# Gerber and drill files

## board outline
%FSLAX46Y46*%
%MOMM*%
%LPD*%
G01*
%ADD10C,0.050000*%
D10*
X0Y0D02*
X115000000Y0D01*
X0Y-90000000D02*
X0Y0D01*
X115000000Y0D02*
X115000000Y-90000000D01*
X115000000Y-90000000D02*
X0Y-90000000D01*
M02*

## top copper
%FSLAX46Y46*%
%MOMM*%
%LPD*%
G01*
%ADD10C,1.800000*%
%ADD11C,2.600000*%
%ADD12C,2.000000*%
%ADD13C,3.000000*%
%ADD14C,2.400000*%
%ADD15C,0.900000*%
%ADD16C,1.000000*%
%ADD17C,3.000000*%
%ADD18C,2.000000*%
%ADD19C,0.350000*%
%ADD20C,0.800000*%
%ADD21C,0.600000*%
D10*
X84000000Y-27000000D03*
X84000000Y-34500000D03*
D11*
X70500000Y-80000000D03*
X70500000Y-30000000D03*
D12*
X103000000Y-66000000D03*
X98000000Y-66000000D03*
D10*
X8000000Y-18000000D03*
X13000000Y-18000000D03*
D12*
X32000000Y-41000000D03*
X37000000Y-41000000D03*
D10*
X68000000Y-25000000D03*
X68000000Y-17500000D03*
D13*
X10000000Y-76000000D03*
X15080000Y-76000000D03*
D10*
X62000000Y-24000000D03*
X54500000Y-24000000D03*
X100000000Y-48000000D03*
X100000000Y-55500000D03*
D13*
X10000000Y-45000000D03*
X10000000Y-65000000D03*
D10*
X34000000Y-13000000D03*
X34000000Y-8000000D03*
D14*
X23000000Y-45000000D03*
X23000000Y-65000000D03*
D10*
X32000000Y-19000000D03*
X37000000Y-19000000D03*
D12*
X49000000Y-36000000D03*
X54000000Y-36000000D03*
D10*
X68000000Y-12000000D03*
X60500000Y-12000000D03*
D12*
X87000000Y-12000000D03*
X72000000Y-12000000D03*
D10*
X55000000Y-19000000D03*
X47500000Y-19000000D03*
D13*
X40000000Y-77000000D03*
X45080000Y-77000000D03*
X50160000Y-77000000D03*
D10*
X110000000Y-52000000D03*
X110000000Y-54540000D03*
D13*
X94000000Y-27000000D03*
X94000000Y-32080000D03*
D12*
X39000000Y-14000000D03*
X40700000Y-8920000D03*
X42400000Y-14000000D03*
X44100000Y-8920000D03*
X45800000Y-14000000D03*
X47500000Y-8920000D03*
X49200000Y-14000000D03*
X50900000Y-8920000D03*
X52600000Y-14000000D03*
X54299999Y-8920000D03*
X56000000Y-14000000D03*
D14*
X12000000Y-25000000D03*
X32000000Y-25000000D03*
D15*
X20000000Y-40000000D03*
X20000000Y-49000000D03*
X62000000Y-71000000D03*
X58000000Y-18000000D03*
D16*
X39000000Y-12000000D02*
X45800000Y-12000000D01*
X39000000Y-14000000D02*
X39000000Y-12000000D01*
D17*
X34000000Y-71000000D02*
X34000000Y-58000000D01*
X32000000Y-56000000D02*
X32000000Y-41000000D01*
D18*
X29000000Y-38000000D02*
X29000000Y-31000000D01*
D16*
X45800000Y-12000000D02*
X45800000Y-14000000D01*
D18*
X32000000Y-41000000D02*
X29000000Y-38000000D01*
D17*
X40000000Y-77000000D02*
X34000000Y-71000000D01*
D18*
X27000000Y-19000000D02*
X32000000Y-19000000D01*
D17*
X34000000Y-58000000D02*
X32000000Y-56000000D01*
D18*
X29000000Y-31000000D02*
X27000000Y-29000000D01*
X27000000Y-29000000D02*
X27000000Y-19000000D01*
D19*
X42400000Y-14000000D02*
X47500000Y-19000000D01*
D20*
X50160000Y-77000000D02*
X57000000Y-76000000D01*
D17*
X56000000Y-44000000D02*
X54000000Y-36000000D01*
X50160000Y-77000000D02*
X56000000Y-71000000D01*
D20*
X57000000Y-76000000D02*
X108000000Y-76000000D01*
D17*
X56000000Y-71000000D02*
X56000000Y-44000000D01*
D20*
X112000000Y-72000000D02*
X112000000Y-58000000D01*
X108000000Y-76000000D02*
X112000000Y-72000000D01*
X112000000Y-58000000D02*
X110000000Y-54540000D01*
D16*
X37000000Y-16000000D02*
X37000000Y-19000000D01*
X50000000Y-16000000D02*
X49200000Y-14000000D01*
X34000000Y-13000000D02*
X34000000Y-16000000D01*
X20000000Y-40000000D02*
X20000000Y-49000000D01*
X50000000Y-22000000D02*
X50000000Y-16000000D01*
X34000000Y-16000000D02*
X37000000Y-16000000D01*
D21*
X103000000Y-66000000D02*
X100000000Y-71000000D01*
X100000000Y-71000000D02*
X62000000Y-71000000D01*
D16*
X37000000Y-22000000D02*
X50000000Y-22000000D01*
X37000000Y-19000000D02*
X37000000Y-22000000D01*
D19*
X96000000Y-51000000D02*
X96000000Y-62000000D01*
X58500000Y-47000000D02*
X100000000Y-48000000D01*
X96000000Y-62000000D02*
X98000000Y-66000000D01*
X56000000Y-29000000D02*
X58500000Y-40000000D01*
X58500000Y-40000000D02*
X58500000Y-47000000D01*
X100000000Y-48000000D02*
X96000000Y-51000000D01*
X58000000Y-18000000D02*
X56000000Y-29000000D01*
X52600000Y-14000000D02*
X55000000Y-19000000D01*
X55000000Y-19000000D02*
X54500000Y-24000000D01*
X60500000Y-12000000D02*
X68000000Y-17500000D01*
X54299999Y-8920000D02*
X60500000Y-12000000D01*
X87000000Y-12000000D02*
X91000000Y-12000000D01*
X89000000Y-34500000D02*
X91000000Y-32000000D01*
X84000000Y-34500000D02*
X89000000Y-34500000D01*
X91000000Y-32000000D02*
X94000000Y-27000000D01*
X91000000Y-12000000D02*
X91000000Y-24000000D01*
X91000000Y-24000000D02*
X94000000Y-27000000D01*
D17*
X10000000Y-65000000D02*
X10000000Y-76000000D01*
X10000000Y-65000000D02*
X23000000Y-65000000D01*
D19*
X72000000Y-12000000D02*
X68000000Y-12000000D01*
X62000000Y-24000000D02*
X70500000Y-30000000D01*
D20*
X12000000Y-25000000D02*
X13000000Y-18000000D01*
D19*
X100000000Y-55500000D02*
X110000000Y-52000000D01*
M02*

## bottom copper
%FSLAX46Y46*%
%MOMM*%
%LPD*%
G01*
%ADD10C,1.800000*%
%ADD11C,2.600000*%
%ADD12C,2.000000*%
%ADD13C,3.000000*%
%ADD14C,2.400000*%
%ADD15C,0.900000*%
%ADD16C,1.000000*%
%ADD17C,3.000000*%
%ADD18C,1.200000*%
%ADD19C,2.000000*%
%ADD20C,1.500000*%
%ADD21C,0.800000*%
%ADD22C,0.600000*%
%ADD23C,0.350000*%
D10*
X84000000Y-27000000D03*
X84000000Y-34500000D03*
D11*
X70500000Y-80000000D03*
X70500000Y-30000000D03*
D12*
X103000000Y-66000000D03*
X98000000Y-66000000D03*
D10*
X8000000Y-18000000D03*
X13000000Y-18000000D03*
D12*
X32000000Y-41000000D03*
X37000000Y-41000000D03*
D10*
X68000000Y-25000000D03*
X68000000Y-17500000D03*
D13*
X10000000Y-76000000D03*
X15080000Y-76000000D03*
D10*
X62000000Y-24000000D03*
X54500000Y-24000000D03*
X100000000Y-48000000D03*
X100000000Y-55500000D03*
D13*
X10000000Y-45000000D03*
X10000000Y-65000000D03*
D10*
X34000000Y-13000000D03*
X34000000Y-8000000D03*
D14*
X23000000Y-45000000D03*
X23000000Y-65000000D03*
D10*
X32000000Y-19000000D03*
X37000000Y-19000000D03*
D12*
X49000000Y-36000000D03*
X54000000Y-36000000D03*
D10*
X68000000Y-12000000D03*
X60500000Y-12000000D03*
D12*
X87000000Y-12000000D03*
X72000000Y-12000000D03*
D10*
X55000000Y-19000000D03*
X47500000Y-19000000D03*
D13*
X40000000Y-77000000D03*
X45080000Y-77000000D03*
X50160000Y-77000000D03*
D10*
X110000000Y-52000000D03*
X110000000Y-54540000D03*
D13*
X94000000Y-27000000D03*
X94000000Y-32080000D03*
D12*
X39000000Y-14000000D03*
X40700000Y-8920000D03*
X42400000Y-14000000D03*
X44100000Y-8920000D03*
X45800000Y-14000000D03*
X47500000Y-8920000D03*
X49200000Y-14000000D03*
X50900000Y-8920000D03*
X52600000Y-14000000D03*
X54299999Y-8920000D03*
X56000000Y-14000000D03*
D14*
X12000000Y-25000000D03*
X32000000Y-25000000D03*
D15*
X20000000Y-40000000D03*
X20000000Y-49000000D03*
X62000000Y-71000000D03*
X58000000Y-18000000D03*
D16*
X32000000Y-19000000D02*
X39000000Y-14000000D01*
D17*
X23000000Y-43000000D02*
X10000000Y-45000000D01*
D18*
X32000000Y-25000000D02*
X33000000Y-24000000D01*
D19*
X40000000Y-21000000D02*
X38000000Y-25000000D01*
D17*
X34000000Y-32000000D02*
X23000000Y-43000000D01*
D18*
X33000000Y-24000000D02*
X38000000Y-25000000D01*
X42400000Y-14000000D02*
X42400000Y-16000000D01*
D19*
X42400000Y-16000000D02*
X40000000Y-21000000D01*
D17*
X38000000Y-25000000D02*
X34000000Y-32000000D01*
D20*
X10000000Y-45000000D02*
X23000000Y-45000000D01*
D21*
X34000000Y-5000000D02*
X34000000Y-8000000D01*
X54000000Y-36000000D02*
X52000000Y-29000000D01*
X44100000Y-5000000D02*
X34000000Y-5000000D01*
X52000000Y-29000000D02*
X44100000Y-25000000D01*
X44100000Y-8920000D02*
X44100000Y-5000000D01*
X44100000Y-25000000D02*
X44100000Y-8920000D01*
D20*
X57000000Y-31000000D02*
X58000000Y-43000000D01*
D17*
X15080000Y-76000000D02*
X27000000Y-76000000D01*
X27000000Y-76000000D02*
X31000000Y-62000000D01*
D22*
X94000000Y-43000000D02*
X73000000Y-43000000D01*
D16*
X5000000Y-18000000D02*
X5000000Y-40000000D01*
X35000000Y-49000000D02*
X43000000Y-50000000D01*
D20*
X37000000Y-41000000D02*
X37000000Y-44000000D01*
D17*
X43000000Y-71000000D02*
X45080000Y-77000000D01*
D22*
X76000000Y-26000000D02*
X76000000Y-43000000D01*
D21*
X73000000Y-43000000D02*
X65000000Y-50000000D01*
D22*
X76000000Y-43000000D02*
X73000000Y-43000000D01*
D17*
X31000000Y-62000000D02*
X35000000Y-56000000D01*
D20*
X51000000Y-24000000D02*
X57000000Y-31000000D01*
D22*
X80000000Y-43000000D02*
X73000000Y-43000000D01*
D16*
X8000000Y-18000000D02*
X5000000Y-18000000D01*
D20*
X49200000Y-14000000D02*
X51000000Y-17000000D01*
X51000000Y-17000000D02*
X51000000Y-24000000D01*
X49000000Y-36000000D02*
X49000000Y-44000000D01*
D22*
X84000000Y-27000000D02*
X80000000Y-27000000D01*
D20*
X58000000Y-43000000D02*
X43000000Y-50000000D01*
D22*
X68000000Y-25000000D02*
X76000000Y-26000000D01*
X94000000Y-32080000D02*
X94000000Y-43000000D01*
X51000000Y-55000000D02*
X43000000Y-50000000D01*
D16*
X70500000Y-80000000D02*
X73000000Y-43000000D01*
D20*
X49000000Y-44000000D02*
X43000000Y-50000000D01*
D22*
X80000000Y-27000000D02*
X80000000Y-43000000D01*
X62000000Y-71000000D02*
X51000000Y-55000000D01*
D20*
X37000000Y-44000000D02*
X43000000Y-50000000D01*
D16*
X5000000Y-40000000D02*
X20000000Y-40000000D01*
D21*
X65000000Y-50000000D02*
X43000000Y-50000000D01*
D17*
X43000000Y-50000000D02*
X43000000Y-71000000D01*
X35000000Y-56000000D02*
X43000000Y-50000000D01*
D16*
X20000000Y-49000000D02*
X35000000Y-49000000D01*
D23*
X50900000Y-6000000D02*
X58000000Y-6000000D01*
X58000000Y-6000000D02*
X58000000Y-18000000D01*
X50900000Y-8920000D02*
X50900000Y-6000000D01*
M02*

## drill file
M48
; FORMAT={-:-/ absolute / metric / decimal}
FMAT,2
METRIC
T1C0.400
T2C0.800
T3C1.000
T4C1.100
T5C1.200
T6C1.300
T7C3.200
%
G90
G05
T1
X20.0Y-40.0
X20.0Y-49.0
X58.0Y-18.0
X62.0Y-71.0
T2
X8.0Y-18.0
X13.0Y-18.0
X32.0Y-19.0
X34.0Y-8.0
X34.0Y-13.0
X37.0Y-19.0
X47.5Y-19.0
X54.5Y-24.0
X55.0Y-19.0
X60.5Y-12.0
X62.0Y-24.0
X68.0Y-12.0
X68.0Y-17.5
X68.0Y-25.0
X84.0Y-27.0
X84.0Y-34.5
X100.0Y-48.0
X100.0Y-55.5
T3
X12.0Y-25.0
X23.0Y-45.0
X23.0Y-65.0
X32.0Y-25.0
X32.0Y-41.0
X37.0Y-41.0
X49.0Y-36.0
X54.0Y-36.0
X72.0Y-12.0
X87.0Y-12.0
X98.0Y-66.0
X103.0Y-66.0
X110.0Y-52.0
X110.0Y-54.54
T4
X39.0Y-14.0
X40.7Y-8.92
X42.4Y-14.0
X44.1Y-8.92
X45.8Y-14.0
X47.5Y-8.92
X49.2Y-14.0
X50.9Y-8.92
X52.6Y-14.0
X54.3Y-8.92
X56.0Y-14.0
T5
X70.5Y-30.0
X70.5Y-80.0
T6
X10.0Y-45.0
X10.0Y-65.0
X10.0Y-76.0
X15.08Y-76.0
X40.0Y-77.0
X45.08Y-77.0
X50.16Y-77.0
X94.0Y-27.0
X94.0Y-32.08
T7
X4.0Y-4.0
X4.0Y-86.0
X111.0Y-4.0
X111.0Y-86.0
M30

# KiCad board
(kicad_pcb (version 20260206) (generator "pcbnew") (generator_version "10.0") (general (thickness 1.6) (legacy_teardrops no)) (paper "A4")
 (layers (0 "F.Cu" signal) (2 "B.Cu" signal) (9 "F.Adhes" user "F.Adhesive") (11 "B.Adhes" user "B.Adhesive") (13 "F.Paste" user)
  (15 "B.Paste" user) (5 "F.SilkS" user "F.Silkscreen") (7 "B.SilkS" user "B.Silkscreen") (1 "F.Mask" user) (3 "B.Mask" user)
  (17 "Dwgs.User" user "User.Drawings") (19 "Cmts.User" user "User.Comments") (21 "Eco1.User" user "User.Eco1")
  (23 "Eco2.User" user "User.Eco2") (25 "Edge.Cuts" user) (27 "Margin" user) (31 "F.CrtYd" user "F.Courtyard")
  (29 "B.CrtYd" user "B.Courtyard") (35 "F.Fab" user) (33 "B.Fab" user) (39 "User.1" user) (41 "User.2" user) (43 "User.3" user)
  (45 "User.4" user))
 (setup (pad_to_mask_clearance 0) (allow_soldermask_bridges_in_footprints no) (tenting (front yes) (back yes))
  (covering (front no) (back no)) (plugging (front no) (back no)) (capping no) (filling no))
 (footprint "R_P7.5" (layer "F.Cu") (at 84 27 -90)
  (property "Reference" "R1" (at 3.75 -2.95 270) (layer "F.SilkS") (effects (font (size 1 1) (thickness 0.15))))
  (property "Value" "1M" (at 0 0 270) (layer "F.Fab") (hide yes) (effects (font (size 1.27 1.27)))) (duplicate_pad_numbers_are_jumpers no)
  (pad "1" thru_hole circle (at 0 0 270) (size 1.8 1.8) (drill 0.8) (layers "*.Cu" "*.Mask") (remove_unused_layers no) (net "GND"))
  (pad "2" thru_hole circle (at 7.5 0 270) (size 1.8 1.8) (drill 0.8) (layers "*.Cu" "*.Mask") (remove_unused_layers no) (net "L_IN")))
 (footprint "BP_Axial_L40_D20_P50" (layer "F.Cu") (at 70.5 80 90)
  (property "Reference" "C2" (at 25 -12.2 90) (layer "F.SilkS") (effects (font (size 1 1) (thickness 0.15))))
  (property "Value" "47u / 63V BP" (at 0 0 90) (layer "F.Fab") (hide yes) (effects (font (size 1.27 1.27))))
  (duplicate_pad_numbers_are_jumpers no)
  (pad "1" thru_hole circle (at 0 0 90) (size 2.6 2.6) (drill 1.2) (layers "*.Cu" "*.Mask") (remove_unused_layers no) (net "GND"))
  (pad "2" thru_hole circle (at 50 0 90) (size 2.6 2.6) (drill 1.2) (layers "*.Cu" "*.Mask") (remove_unused_layers no) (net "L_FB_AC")))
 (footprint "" (layer "F.Cu") (at 111 86)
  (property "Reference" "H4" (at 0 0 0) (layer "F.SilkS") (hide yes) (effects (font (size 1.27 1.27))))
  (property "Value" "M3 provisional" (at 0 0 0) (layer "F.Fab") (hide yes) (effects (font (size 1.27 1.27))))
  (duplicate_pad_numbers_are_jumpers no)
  (pad "" np_thru_hole circle (at 0 0) (size 3.2 3.2) (drill 3.2) (layers "*.Cu" "*.Mask")))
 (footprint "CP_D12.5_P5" (layer "F.Cu") (at 103 66 180)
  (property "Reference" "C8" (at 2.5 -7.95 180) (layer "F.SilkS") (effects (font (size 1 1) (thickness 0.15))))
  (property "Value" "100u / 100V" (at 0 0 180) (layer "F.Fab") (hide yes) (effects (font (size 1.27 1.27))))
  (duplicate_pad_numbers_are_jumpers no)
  (pad "1" thru_hole circle (at 0 0 180) (size 2 2) (drill 1) (layers "*.Cu" "*.Mask") (remove_unused_layers no) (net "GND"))
  (pad "2" thru_hole circle (at 5 0 180) (size 2 2) (drill 1) (layers "*.Cu" "*.Mask") (remove_unused_layers no) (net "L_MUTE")))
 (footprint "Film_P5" (layer "F.Cu") (at 8 18)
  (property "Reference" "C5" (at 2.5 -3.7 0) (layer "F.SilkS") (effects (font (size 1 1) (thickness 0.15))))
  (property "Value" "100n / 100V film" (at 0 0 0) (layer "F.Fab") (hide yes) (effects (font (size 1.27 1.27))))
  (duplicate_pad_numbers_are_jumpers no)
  (pad "1" thru_hole circle (at 0 0) (size 1.8 1.8) (drill 0.8) (layers "*.Cu" "*.Mask") (remove_unused_layers no) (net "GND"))
  (pad "2" thru_hole circle (at 5 0) (size 1.8 1.8) (drill 0.8) (layers "*.Cu" "*.Mask") (remove_unused_layers no) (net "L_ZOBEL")))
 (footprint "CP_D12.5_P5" (layer "F.Cu") (at 32 41)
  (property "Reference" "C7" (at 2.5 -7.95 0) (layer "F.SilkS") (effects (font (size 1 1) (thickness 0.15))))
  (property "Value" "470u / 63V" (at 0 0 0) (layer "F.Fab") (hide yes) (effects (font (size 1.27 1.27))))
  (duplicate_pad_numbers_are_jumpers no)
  (pad "1" thru_hole circle (at 0 0) (size 2 2) (drill 1) (layers "*.Cu" "*.Mask") (remove_unused_layers no) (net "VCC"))
  (pad "2" thru_hole circle (at 5 0) (size 2 2) (drill 1) (layers "*.Cu" "*.Mask") (remove_unused_layers no) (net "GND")))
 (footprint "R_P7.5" (layer "F.Cu") (at 68 25 90)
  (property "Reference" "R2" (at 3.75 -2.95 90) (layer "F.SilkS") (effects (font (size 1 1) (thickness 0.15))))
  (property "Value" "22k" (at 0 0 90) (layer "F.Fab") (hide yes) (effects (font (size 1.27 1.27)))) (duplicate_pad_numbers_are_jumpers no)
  (pad "1" thru_hole circle (at 0 0 90) (size 1.8 1.8) (drill 0.8) (layers "*.Cu" "*.Mask") (remove_unused_layers no) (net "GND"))
  (pad "2" thru_hole circle (at 7.5 0 90) (size 1.8 1.8) (drill 0.8) (layers "*.Cu" "*.Mask") (remove_unused_layers no) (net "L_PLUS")))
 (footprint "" (layer "F.Cu") (at 111 4)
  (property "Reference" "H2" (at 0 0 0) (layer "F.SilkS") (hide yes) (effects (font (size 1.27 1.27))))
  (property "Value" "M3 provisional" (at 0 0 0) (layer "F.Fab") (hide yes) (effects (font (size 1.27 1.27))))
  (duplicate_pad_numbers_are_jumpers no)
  (pad "" np_thru_hole circle (at 0 0) (size 3.2 3.2) (drill 3.2) (layers "*.Cu" "*.Mask")))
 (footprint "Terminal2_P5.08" (layer "F.Cu") (at 10 76)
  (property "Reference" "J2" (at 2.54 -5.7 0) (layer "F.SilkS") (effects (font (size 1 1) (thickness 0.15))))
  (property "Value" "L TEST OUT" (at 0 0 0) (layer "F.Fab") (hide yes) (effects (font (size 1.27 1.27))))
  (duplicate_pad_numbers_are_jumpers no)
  (pad "1" thru_hole circle (at 0 0) (size 3 3) (drill 1.3) (layers "*.Cu" "*.Mask") (remove_unused_layers no) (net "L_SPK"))
  (pad "2" thru_hole circle (at 5.08 0) (size 3 3) (drill 1.3) (layers "*.Cu" "*.Mask") (remove_unused_layers no) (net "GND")))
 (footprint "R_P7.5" (layer "F.Cu") (at 62 24 180)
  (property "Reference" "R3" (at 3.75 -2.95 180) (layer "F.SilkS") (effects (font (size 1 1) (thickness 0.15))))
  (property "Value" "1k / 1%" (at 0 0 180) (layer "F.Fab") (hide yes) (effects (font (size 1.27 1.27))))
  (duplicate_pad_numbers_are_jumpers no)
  (pad "1" thru_hole circle (at 0 0 180) (size 1.8 1.8) (drill 0.8) (layers "*.Cu" "*.Mask") (remove_unused_layers no) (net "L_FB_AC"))
  (pad "2" thru_hole circle (at 7.5 0 180) (size 1.8 1.8) (drill 0.8) (layers "*.Cu" "*.Mask") (remove_unused_layers no) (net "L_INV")))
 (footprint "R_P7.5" (layer "F.Cu") (at 100 48 -90)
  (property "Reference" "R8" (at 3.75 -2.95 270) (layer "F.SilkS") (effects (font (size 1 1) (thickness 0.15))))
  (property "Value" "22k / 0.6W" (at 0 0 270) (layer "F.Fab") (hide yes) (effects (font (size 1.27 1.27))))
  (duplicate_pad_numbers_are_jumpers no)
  (pad "1" thru_hole circle (at 0 0 270) (size 1.8 1.8) (drill 0.8) (layers "*.Cu" "*.Mask") (remove_unused_layers no) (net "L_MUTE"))
  (pad "2" thru_hole circle (at 7.5 0 270) (size 1.8 1.8) (drill 0.8) (layers "*.Cu" "*.Mask") (remove_unused_layers no) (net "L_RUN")))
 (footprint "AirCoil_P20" (layer "F.Cu") (at 10 45 -90)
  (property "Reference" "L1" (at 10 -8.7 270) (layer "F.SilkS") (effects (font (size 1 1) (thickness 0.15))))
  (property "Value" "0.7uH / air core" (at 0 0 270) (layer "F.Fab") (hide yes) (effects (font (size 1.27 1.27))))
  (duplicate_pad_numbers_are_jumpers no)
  (pad "1" thru_hole circle (at 0 0 270) (size 3 3) (drill 1.3) (layers "*.Cu" "*.Mask") (remove_unused_layers no) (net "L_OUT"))
  (pad "2" thru_hole circle (at 20 0 270) (size 3 3) (drill 1.3) (layers "*.Cu" "*.Mask") (remove_unused_layers no) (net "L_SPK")))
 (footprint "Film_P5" (layer "F.Cu") (at 34 13 90)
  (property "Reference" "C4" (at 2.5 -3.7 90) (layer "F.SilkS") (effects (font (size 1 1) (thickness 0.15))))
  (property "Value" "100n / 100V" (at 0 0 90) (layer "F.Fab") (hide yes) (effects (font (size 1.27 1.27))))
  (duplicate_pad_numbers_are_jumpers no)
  (pad "1" thru_hole circle (at 0 0 90) (size 1.8 1.8) (drill 0.8) (layers "*.Cu" "*.Mask") (remove_unused_layers no) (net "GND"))
  (pad "2" thru_hole circle (at 5 0 90) (size 1.8 1.8) (drill 0.8) (layers "*.Cu" "*.Mask") (remove_unused_layers no) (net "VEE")))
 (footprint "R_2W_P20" (layer "F.Cu") (at 23 45 -90)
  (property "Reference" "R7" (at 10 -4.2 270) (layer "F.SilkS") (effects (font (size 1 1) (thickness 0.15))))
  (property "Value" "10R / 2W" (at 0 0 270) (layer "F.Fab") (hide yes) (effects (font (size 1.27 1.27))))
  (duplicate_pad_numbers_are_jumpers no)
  (pad "1" thru_hole circle (at 0 0 270) (size 2.4 2.4) (drill 1) (layers "*.Cu" "*.Mask") (remove_unused_layers no) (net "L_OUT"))
  (pad "2" thru_hole circle (at 20 0 270) (size 2.4 2.4) (drill 1) (layers "*.Cu" "*.Mask") (remove_unused_layers no) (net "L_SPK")))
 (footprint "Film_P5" (layer "F.Cu") (at 32 19)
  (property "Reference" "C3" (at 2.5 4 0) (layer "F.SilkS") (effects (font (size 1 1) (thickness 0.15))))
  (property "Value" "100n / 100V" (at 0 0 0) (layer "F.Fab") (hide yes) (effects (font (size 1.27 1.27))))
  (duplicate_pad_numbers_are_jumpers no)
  (pad "1" thru_hole circle (at 0 0) (size 1.8 1.8) (drill 0.8) (layers "*.Cu" "*.Mask") (remove_unused_layers no) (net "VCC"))
  (pad "2" thru_hole circle (at 5 0) (size 1.8 1.8) (drill 0.8) (layers "*.Cu" "*.Mask") (remove_unused_layers no) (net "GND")))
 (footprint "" (layer "F.Cu") (at 4 86)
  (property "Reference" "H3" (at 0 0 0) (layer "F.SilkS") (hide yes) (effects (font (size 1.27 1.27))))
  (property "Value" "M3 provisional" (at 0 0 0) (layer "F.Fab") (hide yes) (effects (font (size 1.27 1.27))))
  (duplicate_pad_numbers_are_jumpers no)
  (pad "" np_thru_hole circle (at 0 0) (size 3.2 3.2) (drill 3.2) (layers "*.Cu" "*.Mask")))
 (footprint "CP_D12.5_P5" (layer "F.Cu") (at 49 36)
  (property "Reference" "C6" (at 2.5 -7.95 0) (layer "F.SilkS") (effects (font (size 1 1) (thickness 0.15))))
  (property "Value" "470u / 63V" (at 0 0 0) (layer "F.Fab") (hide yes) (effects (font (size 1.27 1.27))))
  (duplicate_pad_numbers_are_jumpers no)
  (pad "1" thru_hole circle (at 0 0) (size 2 2) (drill 1) (layers "*.Cu" "*.Mask") (remove_unused_layers no) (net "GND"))
  (pad "2" thru_hole circle (at 5 0) (size 2 2) (drill 1) (layers "*.Cu" "*.Mask") (remove_unused_layers no) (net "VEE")))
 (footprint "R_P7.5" (layer "F.Cu") (at 68 12 180)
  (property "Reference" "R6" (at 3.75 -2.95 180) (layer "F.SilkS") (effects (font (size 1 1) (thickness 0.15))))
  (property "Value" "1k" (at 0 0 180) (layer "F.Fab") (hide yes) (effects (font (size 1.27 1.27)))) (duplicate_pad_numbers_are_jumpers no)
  (pad "1" thru_hole circle (at 0 0 180) (size 1.8 1.8) (drill 0.8) (layers "*.Cu" "*.Mask") (remove_unused_layers no) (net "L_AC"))
  (pad "2" thru_hole circle (at 7.5 0 180) (size 1.8 1.8) (drill 0.8) (layers "*.Cu" "*.Mask") (remove_unused_layers no) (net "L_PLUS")))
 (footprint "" (layer "F.Cu") (at 4 4)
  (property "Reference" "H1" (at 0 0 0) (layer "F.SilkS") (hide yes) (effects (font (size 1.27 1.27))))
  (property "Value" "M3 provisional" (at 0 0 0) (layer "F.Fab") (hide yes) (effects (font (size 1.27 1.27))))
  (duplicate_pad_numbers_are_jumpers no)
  (pad "" np_thru_hole circle (at 0 0) (size 3.2 3.2) (drill 3.2) (layers "*.Cu" "*.Mask")))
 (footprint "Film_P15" (layer "F.Cu") (at 87 12 180)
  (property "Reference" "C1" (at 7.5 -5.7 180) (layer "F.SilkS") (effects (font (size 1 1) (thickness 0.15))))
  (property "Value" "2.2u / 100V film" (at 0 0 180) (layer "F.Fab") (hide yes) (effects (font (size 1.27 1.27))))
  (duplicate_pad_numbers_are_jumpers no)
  (pad "1" thru_hole circle (at 0 0 180) (size 2 2) (drill 1) (layers "*.Cu" "*.Mask") (remove_unused_layers no) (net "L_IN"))
  (pad "2" thru_hole circle (at 15 0 180) (size 2 2) (drill 1) (layers "*.Cu" "*.Mask") (remove_unused_layers no) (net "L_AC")))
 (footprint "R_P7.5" (layer "F.Cu") (at 55 19 180)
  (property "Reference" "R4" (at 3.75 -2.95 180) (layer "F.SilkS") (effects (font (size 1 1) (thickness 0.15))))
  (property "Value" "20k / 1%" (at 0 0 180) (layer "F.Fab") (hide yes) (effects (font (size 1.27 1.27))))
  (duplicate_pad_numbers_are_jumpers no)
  (pad "1" thru_hole circle (at 0 0 180) (size 1.8 1.8) (drill 0.8) (layers "*.Cu" "*.Mask") (remove_unused_layers no) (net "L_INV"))
  (pad "2" thru_hole circle (at 7.5 0 180) (size 1.8 1.8) (drill 0.8) (layers "*.Cu" "*.Mask") (remove_unused_layers no) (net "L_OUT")))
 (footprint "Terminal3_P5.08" (layer "F.Cu") (at 40 77)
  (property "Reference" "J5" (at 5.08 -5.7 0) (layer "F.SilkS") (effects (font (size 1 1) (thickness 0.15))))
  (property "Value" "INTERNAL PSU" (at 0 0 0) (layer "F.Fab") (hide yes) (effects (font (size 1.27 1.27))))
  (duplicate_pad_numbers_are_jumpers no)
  (pad "1" thru_hole circle (at 0 0) (size 3 3) (drill 1.3) (layers "*.Cu" "*.Mask") (remove_unused_layers no) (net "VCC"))
  (pad "2" thru_hole circle (at 5.08 0) (size 3 3) (drill 1.3) (layers "*.Cu" "*.Mask") (remove_unused_layers no) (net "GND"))
  (pad "3" thru_hole circle (at 10.16 0) (size 3 3) (drill 1.3) (layers "*.Cu" "*.Mask") (remove_unused_layers no) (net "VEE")))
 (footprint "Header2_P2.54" (layer "F.Cu") (at 110 52 -90)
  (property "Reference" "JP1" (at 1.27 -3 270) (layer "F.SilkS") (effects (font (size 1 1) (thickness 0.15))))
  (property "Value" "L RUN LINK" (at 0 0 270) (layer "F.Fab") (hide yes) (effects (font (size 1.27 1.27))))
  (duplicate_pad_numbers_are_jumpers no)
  (pad "1" thru_hole circle (at 0 0 270) (size 1.8 1.8) (drill 1) (layers "*.Cu" "*.Mask") (remove_unused_layers no) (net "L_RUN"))
  (pad "2" thru_hole circle (at 2.54 0 270) (size 1.8 1.8) (drill 1) (layers "*.Cu" "*.Mask") (remove_unused_layers no) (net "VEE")))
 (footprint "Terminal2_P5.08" (layer "F.Cu") (at 94 27 -90)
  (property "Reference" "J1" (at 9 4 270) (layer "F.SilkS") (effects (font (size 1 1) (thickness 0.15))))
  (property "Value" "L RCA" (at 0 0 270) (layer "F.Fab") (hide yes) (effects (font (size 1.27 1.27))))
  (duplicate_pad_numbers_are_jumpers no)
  (pad "1" thru_hole circle (at 0 0 270) (size 3 3) (drill 1.3) (layers "*.Cu" "*.Mask") (remove_unused_layers no) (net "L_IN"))
  (pad "2" thru_hole circle (at 5.08 0 270) (size 3 3) (drill 1.3) (layers "*.Cu" "*.Mask") (remove_unused_layers no) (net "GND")))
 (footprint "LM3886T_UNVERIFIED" (layer "F.Cu") (at 39 14)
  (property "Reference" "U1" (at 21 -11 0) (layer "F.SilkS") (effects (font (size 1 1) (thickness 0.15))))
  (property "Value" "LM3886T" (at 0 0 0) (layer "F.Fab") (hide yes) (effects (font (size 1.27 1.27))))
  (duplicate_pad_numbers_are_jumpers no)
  (pad "1" thru_hole circle (at 0 0) (size 2 2) (drill 1.1) (layers "*.Cu" "*.Mask") (remove_unused_layers no) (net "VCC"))
  (pad "2" thru_hole circle (at 1.7 -5.08) (size 2 2) (drill 1.1) (layers "*.Cu" "*.Mask") (remove_unused_layers no)
   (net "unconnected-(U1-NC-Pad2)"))
  (pad "3" thru_hole circle (at 3.4 0) (size 2 2) (drill 1.1) (layers "*.Cu" "*.Mask") (remove_unused_layers no) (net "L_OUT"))
  (pad "4" thru_hole circle (at 5.1 -5.08) (size 2 2) (drill 1.1) (layers "*.Cu" "*.Mask") (remove_unused_layers no) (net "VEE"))
  (pad "5" thru_hole circle (at 6.8 0) (size 2 2) (drill 1.1) (layers "*.Cu" "*.Mask") (remove_unused_layers no) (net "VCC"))
  (pad "6" thru_hole circle (at 8.5 -5.08) (size 2 2) (drill 1.1) (layers "*.Cu" "*.Mask") (remove_unused_layers no)
   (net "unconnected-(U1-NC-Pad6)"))
  (pad "7" thru_hole circle (at 10.2 0) (size 2 2) (drill 1.1) (layers "*.Cu" "*.Mask") (remove_unused_layers no) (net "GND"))
  (pad "8" thru_hole circle (at 11.9 -5.08) (size 2 2) (drill 1.1) (layers "*.Cu" "*.Mask") (remove_unused_layers no) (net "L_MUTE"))
  (pad "9" thru_hole circle (at 13.6 0) (size 2 2) (drill 1.1) (layers "*.Cu" "*.Mask") (remove_unused_layers no) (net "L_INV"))
  (pad "10" thru_hole circle (at 15.299999 -5.08) (size 2 2) (drill 1.1) (layers "*.Cu" "*.Mask") (remove_unused_layers no) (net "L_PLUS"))
  (pad "11" thru_hole circle (at 17 0) (size 2 2) (drill 1.1) (layers "*.Cu" "*.Mask") (remove_unused_layers no)
   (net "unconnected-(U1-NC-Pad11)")))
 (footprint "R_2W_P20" (layer "F.Cu") (at 12 25)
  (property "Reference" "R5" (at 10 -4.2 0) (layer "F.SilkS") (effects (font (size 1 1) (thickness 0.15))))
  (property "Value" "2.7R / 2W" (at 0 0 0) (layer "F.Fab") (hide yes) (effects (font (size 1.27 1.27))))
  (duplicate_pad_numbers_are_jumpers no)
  (pad "1" thru_hole circle (at 0 0) (size 2.4 2.4) (drill 1) (layers "*.Cu" "*.Mask") (remove_unused_layers no) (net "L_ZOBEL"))
  (pad "2" thru_hole circle (at 20 0) (size 2.4 2.4) (drill 1) (layers "*.Cu" "*.Mask") (remove_unused_layers no) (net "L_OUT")))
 (gr_line (start 0 0) (end 115 0) (stroke (width 0.05) (type default)) (layer "Edge.Cuts"))
 (gr_line (start 0 90) (end 0 0) (stroke (width 0.05) (type default)) (layer "Edge.Cuts"))
 (gr_line (start 115 0) (end 115 90) (stroke (width 0.05) (type default)) (layer "Edge.Cuts"))
 (gr_line (start 115 90) (end 0 90) (stroke (width 0.05) (type default)) (layer "Edge.Cuts"))
 (segment (start 39 12) (end 45.8 12) (width 1) (layer "F.Cu") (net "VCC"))
 (segment (start 39 14) (end 39 12) (width 1) (layer "F.Cu") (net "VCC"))
 (segment (start 34 71) (end 34 58) (width 3) (layer "F.Cu") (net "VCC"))
 (segment (start 32 56) (end 32 41) (width 3) (layer "F.Cu") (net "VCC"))
 (segment (start 29 38) (end 29 31) (width 2) (layer "F.Cu") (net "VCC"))
 (segment (start 45.8 12) (end 45.8 14) (width 1) (layer "F.Cu") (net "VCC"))
 (segment (start 32 41) (end 29 38) (width 2) (layer "F.Cu") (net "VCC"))
 (segment (start 40 77) (end 34 71) (width 3) (layer "F.Cu") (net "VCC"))
 (segment (start 27 19) (end 32 19) (width 2) (layer "F.Cu") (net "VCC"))
 (segment (start 34 58) (end 32 56) (width 3) (layer "F.Cu") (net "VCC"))
 (segment (start 29 31) (end 27 29) (width 2) (layer "F.Cu") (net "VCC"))
 (segment (start 27 29) (end 27 19) (width 2) (layer "F.Cu") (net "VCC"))
 (segment (start 32 19) (end 39 14) (width 1) (layer "B.Cu") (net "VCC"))
 (segment (start 42.4 14) (end 47.5 19) (width 0.35) (layer "F.Cu") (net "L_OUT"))
 (segment (start 23 43) (end 10 45) (width 3) (layer "B.Cu") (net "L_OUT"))
 (segment (start 32 25) (end 33 24) (width 1.2) (layer "B.Cu") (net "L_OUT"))
 (segment (start 40 21) (end 38 25) (width 2) (layer "B.Cu") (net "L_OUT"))
 (segment (start 34 32) (end 23 43) (width 3) (layer "B.Cu") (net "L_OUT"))
 (segment (start 33 24) (end 38 25) (width 1.2) (layer "B.Cu") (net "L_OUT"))
 (segment (start 42.4 14) (end 42.4 16) (width 1.2) (layer "B.Cu") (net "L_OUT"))
 (segment (start 42.4 16) (end 40 21) (width 2) (layer "B.Cu") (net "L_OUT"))
 (segment (start 38 25) (end 34 32) (width 3) (layer "B.Cu") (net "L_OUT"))
 (segment (start 10 45) (end 23 45) (width 1.5) (layer "B.Cu") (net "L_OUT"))
 (segment (start 50.16 77) (end 57 76) (width 0.8) (layer "F.Cu") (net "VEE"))
 (segment (start 56 44) (end 54 36) (width 3) (layer "F.Cu") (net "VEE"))
 (segment (start 50.16 77) (end 56 71) (width 3) (layer "F.Cu") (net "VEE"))
 (segment (start 57 76) (end 108 76) (width 0.8) (layer "F.Cu") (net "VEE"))
 (segment (start 56 71) (end 56 44) (width 3) (layer "F.Cu") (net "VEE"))
 (segment (start 112 72) (end 112 58) (width 0.8) (layer "F.Cu") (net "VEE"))
 (segment (start 108 76) (end 112 72) (width 0.8) (layer "F.Cu") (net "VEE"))
 (segment (start 112 58) (end 110 54.54) (width 0.8) (layer "F.Cu") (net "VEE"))
 (segment (start 34 5) (end 34 8) (width 0.8) (layer "B.Cu") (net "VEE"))
 (segment (start 54 36) (end 52 29) (width 0.8) (layer "B.Cu") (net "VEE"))
 (segment (start 44.1 5) (end 34 5) (width 0.8) (layer "B.Cu") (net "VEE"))
 (segment (start 52 29) (end 44.1 25) (width 0.8) (layer "B.Cu") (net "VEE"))
 (segment (start 44.1 8.92) (end 44.1 5) (width 0.8) (layer "B.Cu") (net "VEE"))
 (segment (start 44.1 25) (end 44.1 8.92) (width 0.8) (layer "B.Cu") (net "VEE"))
 (segment (start 37 16) (end 37 19) (width 1) (layer "F.Cu") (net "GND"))
 (segment (start 50 16) (end 49.2 14) (width 1) (layer "F.Cu") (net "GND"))
 (segment (start 34 13) (end 34 16) (width 1) (layer "F.Cu") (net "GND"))
 (segment (start 20 40) (end 20 49) (width 1) (layer "F.Cu") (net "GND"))
 (segment (start 50 22) (end 50 16) (width 1) (layer "F.Cu") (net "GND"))
 (segment (start 34 16) (end 37 16) (width 1) (layer "F.Cu") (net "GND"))
 (segment (start 103 66) (end 100 71) (width 0.6) (layer "F.Cu") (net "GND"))
 (segment (start 100 71) (end 62 71) (width 0.6) (layer "F.Cu") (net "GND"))
 (segment (start 37 22) (end 50 22) (width 1) (layer "F.Cu") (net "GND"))
 (segment (start 37 19) (end 37 22) (width 1) (layer "F.Cu") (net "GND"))
 (via (at 20 40) (size 0.9) (drill 0.4) (layers "F.Cu" "B.Cu") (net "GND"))
 (via (at 20 49) (size 0.9) (drill 0.4) (layers "F.Cu" "B.Cu") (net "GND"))
 (via (at 62 71) (size 0.9) (drill 0.4) (layers "F.Cu" "B.Cu") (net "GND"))
 (segment (start 57 31) (end 58 43) (width 1.5) (layer "B.Cu") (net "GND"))
 (segment (start 15.08 76) (end 27 76) (width 3) (layer "B.Cu") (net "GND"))
 (segment (start 27 76) (end 31 62) (width 3) (layer "B.Cu") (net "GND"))
 (segment (start 94 43) (end 73 43) (width 0.6) (layer "B.Cu") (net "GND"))
 (segment (start 5 18) (end 5 40) (width 1) (layer "B.Cu") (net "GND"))
 (segment (start 35 49) (end 43 50) (width 1) (layer "B.Cu") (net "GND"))
 (segment (start 37 41) (end 37 44) (width 1.5) (layer "B.Cu") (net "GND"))
 (segment (start 43 71) (end 45.08 77) (width 3) (layer "B.Cu") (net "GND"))
 (segment (start 76 26) (end 76 43) (width 0.6) (layer "B.Cu") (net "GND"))
 (segment (start 73 43) (end 65 50) (width 0.8) (layer "B.Cu") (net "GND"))
 (segment (start 76 43) (end 73 43) (width 0.6) (layer "B.Cu") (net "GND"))
 (segment (start 31 62) (end 35 56) (width 3) (layer "B.Cu") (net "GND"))
 (segment (start 51 24) (end 57 31) (width 1.5) (layer "B.Cu") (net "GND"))
 (segment (start 80 43) (end 73 43) (width 0.6) (layer "B.Cu") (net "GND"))
 (segment (start 8 18) (end 5 18) (width 1) (layer "B.Cu") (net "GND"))
 (segment (start 49.2 14) (end 51 17) (width 1.5) (layer "B.Cu") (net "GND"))
 (segment (start 51 17) (end 51 24) (width 1.5) (layer "B.Cu") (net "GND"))
 (segment (start 49 36) (end 49 44) (width 1.5) (layer "B.Cu") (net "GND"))
 (segment (start 84 27) (end 80 27) (width 0.6) (layer "B.Cu") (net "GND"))
 (segment (start 58 43) (end 43 50) (width 1.5) (layer "B.Cu") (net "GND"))
 (segment (start 68 25) (end 76 26) (width 0.6) (layer "B.Cu") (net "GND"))
 (segment (start 94 32.08) (end 94 43) (width 0.6) (layer "B.Cu") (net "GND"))
 (segment (start 51 55) (end 43 50) (width 0.6) (layer "B.Cu") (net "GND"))
 (segment (start 70.5 80) (end 73 43) (width 1) (layer "B.Cu") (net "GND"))
 (segment (start 49 44) (end 43 50) (width 1.5) (layer "B.Cu") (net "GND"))
 (segment (start 80 27) (end 80 43) (width 0.6) (layer "B.Cu") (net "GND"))
 (segment (start 62 71) (end 51 55) (width 0.6) (layer "B.Cu") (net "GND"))
 (segment (start 37 44) (end 43 50) (width 1.5) (layer "B.Cu") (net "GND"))
 (segment (start 5 40) (end 20 40) (width 1) (layer "B.Cu") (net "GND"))
 (segment (start 65 50) (end 43 50) (width 0.8) (layer "B.Cu") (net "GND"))
 (segment (start 43 50) (end 43 71) (width 3) (layer "B.Cu") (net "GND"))
 (segment (start 35 56) (end 43 50) (width 3) (layer "B.Cu") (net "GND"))
 (segment (start 20 49) (end 35 49) (width 1) (layer "B.Cu") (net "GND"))
 (segment (start 96 51) (end 96 62) (width 0.35) (layer "F.Cu") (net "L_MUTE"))
 (segment (start 58.5 47) (end 100 48) (width 0.35) (layer "F.Cu") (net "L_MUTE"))
 (segment (start 96 62) (end 98 66) (width 0.35) (layer "F.Cu") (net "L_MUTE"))
 (segment (start 56 29) (end 58.5 40) (width 0.35) (layer "F.Cu") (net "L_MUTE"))
 (segment (start 58.5 40) (end 58.5 47) (width 0.35) (layer "F.Cu") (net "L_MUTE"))
 (segment (start 100 48) (end 96 51) (width 0.35) (layer "F.Cu") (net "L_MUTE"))
 (segment (start 58 18) (end 56 29) (width 0.35) (layer "F.Cu") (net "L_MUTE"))
 (via (at 58 18) (size 0.9) (drill 0.4) (layers "F.Cu" "B.Cu") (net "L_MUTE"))
 (segment (start 50.9 6) (end 58 6) (width 0.35) (layer "B.Cu") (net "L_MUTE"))
 (segment (start 58 6) (end 58 18) (width 0.35) (layer "B.Cu") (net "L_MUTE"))
 (segment (start 50.9 8.92) (end 50.9 6) (width 0.35) (layer "B.Cu") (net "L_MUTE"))
 (segment (start 52.6 14) (end 55 19) (width 0.35) (layer "F.Cu") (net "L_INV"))
 (segment (start 55 19) (end 54.5 24) (width 0.35) (layer "F.Cu") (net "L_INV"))
 (segment (start 60.5 12) (end 68 17.5) (width 0.35) (layer "F.Cu") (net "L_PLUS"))
 (segment (start 54.299999 8.92) (end 60.5 12) (width 0.35) (layer "F.Cu") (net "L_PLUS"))
 (segment (start 87 12) (end 91 12) (width 0.35) (layer "F.Cu") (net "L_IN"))
 (segment (start 89 34.5) (end 91 32) (width 0.35) (layer "F.Cu") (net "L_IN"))
 (segment (start 84 34.5) (end 89 34.5) (width 0.35) (layer "F.Cu") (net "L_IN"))
 (segment (start 91 32) (end 94 27) (width 0.35) (layer "F.Cu") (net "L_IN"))
 (segment (start 91 12) (end 91 24) (width 0.35) (layer "F.Cu") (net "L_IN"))
 (segment (start 91 24) (end 94 27) (width 0.35) (layer "F.Cu") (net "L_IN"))
 (segment (start 10 65) (end 10 76) (width 3) (layer "F.Cu") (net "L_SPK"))
 (segment (start 10 65) (end 23 65) (width 3) (layer "F.Cu") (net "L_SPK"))
 (segment (start 72 12) (end 68 12) (width 0.35) (layer "F.Cu") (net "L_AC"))
 (segment (start 62 24) (end 70.5 30) (width 0.35) (layer "F.Cu") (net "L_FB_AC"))
 (segment (start 12 25) (end 13 18) (width 0.8) (layer "F.Cu") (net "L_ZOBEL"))
 (segment (start 100 55.5) (end 110 52) (width 0.35) (layer "F.Cu") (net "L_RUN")))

